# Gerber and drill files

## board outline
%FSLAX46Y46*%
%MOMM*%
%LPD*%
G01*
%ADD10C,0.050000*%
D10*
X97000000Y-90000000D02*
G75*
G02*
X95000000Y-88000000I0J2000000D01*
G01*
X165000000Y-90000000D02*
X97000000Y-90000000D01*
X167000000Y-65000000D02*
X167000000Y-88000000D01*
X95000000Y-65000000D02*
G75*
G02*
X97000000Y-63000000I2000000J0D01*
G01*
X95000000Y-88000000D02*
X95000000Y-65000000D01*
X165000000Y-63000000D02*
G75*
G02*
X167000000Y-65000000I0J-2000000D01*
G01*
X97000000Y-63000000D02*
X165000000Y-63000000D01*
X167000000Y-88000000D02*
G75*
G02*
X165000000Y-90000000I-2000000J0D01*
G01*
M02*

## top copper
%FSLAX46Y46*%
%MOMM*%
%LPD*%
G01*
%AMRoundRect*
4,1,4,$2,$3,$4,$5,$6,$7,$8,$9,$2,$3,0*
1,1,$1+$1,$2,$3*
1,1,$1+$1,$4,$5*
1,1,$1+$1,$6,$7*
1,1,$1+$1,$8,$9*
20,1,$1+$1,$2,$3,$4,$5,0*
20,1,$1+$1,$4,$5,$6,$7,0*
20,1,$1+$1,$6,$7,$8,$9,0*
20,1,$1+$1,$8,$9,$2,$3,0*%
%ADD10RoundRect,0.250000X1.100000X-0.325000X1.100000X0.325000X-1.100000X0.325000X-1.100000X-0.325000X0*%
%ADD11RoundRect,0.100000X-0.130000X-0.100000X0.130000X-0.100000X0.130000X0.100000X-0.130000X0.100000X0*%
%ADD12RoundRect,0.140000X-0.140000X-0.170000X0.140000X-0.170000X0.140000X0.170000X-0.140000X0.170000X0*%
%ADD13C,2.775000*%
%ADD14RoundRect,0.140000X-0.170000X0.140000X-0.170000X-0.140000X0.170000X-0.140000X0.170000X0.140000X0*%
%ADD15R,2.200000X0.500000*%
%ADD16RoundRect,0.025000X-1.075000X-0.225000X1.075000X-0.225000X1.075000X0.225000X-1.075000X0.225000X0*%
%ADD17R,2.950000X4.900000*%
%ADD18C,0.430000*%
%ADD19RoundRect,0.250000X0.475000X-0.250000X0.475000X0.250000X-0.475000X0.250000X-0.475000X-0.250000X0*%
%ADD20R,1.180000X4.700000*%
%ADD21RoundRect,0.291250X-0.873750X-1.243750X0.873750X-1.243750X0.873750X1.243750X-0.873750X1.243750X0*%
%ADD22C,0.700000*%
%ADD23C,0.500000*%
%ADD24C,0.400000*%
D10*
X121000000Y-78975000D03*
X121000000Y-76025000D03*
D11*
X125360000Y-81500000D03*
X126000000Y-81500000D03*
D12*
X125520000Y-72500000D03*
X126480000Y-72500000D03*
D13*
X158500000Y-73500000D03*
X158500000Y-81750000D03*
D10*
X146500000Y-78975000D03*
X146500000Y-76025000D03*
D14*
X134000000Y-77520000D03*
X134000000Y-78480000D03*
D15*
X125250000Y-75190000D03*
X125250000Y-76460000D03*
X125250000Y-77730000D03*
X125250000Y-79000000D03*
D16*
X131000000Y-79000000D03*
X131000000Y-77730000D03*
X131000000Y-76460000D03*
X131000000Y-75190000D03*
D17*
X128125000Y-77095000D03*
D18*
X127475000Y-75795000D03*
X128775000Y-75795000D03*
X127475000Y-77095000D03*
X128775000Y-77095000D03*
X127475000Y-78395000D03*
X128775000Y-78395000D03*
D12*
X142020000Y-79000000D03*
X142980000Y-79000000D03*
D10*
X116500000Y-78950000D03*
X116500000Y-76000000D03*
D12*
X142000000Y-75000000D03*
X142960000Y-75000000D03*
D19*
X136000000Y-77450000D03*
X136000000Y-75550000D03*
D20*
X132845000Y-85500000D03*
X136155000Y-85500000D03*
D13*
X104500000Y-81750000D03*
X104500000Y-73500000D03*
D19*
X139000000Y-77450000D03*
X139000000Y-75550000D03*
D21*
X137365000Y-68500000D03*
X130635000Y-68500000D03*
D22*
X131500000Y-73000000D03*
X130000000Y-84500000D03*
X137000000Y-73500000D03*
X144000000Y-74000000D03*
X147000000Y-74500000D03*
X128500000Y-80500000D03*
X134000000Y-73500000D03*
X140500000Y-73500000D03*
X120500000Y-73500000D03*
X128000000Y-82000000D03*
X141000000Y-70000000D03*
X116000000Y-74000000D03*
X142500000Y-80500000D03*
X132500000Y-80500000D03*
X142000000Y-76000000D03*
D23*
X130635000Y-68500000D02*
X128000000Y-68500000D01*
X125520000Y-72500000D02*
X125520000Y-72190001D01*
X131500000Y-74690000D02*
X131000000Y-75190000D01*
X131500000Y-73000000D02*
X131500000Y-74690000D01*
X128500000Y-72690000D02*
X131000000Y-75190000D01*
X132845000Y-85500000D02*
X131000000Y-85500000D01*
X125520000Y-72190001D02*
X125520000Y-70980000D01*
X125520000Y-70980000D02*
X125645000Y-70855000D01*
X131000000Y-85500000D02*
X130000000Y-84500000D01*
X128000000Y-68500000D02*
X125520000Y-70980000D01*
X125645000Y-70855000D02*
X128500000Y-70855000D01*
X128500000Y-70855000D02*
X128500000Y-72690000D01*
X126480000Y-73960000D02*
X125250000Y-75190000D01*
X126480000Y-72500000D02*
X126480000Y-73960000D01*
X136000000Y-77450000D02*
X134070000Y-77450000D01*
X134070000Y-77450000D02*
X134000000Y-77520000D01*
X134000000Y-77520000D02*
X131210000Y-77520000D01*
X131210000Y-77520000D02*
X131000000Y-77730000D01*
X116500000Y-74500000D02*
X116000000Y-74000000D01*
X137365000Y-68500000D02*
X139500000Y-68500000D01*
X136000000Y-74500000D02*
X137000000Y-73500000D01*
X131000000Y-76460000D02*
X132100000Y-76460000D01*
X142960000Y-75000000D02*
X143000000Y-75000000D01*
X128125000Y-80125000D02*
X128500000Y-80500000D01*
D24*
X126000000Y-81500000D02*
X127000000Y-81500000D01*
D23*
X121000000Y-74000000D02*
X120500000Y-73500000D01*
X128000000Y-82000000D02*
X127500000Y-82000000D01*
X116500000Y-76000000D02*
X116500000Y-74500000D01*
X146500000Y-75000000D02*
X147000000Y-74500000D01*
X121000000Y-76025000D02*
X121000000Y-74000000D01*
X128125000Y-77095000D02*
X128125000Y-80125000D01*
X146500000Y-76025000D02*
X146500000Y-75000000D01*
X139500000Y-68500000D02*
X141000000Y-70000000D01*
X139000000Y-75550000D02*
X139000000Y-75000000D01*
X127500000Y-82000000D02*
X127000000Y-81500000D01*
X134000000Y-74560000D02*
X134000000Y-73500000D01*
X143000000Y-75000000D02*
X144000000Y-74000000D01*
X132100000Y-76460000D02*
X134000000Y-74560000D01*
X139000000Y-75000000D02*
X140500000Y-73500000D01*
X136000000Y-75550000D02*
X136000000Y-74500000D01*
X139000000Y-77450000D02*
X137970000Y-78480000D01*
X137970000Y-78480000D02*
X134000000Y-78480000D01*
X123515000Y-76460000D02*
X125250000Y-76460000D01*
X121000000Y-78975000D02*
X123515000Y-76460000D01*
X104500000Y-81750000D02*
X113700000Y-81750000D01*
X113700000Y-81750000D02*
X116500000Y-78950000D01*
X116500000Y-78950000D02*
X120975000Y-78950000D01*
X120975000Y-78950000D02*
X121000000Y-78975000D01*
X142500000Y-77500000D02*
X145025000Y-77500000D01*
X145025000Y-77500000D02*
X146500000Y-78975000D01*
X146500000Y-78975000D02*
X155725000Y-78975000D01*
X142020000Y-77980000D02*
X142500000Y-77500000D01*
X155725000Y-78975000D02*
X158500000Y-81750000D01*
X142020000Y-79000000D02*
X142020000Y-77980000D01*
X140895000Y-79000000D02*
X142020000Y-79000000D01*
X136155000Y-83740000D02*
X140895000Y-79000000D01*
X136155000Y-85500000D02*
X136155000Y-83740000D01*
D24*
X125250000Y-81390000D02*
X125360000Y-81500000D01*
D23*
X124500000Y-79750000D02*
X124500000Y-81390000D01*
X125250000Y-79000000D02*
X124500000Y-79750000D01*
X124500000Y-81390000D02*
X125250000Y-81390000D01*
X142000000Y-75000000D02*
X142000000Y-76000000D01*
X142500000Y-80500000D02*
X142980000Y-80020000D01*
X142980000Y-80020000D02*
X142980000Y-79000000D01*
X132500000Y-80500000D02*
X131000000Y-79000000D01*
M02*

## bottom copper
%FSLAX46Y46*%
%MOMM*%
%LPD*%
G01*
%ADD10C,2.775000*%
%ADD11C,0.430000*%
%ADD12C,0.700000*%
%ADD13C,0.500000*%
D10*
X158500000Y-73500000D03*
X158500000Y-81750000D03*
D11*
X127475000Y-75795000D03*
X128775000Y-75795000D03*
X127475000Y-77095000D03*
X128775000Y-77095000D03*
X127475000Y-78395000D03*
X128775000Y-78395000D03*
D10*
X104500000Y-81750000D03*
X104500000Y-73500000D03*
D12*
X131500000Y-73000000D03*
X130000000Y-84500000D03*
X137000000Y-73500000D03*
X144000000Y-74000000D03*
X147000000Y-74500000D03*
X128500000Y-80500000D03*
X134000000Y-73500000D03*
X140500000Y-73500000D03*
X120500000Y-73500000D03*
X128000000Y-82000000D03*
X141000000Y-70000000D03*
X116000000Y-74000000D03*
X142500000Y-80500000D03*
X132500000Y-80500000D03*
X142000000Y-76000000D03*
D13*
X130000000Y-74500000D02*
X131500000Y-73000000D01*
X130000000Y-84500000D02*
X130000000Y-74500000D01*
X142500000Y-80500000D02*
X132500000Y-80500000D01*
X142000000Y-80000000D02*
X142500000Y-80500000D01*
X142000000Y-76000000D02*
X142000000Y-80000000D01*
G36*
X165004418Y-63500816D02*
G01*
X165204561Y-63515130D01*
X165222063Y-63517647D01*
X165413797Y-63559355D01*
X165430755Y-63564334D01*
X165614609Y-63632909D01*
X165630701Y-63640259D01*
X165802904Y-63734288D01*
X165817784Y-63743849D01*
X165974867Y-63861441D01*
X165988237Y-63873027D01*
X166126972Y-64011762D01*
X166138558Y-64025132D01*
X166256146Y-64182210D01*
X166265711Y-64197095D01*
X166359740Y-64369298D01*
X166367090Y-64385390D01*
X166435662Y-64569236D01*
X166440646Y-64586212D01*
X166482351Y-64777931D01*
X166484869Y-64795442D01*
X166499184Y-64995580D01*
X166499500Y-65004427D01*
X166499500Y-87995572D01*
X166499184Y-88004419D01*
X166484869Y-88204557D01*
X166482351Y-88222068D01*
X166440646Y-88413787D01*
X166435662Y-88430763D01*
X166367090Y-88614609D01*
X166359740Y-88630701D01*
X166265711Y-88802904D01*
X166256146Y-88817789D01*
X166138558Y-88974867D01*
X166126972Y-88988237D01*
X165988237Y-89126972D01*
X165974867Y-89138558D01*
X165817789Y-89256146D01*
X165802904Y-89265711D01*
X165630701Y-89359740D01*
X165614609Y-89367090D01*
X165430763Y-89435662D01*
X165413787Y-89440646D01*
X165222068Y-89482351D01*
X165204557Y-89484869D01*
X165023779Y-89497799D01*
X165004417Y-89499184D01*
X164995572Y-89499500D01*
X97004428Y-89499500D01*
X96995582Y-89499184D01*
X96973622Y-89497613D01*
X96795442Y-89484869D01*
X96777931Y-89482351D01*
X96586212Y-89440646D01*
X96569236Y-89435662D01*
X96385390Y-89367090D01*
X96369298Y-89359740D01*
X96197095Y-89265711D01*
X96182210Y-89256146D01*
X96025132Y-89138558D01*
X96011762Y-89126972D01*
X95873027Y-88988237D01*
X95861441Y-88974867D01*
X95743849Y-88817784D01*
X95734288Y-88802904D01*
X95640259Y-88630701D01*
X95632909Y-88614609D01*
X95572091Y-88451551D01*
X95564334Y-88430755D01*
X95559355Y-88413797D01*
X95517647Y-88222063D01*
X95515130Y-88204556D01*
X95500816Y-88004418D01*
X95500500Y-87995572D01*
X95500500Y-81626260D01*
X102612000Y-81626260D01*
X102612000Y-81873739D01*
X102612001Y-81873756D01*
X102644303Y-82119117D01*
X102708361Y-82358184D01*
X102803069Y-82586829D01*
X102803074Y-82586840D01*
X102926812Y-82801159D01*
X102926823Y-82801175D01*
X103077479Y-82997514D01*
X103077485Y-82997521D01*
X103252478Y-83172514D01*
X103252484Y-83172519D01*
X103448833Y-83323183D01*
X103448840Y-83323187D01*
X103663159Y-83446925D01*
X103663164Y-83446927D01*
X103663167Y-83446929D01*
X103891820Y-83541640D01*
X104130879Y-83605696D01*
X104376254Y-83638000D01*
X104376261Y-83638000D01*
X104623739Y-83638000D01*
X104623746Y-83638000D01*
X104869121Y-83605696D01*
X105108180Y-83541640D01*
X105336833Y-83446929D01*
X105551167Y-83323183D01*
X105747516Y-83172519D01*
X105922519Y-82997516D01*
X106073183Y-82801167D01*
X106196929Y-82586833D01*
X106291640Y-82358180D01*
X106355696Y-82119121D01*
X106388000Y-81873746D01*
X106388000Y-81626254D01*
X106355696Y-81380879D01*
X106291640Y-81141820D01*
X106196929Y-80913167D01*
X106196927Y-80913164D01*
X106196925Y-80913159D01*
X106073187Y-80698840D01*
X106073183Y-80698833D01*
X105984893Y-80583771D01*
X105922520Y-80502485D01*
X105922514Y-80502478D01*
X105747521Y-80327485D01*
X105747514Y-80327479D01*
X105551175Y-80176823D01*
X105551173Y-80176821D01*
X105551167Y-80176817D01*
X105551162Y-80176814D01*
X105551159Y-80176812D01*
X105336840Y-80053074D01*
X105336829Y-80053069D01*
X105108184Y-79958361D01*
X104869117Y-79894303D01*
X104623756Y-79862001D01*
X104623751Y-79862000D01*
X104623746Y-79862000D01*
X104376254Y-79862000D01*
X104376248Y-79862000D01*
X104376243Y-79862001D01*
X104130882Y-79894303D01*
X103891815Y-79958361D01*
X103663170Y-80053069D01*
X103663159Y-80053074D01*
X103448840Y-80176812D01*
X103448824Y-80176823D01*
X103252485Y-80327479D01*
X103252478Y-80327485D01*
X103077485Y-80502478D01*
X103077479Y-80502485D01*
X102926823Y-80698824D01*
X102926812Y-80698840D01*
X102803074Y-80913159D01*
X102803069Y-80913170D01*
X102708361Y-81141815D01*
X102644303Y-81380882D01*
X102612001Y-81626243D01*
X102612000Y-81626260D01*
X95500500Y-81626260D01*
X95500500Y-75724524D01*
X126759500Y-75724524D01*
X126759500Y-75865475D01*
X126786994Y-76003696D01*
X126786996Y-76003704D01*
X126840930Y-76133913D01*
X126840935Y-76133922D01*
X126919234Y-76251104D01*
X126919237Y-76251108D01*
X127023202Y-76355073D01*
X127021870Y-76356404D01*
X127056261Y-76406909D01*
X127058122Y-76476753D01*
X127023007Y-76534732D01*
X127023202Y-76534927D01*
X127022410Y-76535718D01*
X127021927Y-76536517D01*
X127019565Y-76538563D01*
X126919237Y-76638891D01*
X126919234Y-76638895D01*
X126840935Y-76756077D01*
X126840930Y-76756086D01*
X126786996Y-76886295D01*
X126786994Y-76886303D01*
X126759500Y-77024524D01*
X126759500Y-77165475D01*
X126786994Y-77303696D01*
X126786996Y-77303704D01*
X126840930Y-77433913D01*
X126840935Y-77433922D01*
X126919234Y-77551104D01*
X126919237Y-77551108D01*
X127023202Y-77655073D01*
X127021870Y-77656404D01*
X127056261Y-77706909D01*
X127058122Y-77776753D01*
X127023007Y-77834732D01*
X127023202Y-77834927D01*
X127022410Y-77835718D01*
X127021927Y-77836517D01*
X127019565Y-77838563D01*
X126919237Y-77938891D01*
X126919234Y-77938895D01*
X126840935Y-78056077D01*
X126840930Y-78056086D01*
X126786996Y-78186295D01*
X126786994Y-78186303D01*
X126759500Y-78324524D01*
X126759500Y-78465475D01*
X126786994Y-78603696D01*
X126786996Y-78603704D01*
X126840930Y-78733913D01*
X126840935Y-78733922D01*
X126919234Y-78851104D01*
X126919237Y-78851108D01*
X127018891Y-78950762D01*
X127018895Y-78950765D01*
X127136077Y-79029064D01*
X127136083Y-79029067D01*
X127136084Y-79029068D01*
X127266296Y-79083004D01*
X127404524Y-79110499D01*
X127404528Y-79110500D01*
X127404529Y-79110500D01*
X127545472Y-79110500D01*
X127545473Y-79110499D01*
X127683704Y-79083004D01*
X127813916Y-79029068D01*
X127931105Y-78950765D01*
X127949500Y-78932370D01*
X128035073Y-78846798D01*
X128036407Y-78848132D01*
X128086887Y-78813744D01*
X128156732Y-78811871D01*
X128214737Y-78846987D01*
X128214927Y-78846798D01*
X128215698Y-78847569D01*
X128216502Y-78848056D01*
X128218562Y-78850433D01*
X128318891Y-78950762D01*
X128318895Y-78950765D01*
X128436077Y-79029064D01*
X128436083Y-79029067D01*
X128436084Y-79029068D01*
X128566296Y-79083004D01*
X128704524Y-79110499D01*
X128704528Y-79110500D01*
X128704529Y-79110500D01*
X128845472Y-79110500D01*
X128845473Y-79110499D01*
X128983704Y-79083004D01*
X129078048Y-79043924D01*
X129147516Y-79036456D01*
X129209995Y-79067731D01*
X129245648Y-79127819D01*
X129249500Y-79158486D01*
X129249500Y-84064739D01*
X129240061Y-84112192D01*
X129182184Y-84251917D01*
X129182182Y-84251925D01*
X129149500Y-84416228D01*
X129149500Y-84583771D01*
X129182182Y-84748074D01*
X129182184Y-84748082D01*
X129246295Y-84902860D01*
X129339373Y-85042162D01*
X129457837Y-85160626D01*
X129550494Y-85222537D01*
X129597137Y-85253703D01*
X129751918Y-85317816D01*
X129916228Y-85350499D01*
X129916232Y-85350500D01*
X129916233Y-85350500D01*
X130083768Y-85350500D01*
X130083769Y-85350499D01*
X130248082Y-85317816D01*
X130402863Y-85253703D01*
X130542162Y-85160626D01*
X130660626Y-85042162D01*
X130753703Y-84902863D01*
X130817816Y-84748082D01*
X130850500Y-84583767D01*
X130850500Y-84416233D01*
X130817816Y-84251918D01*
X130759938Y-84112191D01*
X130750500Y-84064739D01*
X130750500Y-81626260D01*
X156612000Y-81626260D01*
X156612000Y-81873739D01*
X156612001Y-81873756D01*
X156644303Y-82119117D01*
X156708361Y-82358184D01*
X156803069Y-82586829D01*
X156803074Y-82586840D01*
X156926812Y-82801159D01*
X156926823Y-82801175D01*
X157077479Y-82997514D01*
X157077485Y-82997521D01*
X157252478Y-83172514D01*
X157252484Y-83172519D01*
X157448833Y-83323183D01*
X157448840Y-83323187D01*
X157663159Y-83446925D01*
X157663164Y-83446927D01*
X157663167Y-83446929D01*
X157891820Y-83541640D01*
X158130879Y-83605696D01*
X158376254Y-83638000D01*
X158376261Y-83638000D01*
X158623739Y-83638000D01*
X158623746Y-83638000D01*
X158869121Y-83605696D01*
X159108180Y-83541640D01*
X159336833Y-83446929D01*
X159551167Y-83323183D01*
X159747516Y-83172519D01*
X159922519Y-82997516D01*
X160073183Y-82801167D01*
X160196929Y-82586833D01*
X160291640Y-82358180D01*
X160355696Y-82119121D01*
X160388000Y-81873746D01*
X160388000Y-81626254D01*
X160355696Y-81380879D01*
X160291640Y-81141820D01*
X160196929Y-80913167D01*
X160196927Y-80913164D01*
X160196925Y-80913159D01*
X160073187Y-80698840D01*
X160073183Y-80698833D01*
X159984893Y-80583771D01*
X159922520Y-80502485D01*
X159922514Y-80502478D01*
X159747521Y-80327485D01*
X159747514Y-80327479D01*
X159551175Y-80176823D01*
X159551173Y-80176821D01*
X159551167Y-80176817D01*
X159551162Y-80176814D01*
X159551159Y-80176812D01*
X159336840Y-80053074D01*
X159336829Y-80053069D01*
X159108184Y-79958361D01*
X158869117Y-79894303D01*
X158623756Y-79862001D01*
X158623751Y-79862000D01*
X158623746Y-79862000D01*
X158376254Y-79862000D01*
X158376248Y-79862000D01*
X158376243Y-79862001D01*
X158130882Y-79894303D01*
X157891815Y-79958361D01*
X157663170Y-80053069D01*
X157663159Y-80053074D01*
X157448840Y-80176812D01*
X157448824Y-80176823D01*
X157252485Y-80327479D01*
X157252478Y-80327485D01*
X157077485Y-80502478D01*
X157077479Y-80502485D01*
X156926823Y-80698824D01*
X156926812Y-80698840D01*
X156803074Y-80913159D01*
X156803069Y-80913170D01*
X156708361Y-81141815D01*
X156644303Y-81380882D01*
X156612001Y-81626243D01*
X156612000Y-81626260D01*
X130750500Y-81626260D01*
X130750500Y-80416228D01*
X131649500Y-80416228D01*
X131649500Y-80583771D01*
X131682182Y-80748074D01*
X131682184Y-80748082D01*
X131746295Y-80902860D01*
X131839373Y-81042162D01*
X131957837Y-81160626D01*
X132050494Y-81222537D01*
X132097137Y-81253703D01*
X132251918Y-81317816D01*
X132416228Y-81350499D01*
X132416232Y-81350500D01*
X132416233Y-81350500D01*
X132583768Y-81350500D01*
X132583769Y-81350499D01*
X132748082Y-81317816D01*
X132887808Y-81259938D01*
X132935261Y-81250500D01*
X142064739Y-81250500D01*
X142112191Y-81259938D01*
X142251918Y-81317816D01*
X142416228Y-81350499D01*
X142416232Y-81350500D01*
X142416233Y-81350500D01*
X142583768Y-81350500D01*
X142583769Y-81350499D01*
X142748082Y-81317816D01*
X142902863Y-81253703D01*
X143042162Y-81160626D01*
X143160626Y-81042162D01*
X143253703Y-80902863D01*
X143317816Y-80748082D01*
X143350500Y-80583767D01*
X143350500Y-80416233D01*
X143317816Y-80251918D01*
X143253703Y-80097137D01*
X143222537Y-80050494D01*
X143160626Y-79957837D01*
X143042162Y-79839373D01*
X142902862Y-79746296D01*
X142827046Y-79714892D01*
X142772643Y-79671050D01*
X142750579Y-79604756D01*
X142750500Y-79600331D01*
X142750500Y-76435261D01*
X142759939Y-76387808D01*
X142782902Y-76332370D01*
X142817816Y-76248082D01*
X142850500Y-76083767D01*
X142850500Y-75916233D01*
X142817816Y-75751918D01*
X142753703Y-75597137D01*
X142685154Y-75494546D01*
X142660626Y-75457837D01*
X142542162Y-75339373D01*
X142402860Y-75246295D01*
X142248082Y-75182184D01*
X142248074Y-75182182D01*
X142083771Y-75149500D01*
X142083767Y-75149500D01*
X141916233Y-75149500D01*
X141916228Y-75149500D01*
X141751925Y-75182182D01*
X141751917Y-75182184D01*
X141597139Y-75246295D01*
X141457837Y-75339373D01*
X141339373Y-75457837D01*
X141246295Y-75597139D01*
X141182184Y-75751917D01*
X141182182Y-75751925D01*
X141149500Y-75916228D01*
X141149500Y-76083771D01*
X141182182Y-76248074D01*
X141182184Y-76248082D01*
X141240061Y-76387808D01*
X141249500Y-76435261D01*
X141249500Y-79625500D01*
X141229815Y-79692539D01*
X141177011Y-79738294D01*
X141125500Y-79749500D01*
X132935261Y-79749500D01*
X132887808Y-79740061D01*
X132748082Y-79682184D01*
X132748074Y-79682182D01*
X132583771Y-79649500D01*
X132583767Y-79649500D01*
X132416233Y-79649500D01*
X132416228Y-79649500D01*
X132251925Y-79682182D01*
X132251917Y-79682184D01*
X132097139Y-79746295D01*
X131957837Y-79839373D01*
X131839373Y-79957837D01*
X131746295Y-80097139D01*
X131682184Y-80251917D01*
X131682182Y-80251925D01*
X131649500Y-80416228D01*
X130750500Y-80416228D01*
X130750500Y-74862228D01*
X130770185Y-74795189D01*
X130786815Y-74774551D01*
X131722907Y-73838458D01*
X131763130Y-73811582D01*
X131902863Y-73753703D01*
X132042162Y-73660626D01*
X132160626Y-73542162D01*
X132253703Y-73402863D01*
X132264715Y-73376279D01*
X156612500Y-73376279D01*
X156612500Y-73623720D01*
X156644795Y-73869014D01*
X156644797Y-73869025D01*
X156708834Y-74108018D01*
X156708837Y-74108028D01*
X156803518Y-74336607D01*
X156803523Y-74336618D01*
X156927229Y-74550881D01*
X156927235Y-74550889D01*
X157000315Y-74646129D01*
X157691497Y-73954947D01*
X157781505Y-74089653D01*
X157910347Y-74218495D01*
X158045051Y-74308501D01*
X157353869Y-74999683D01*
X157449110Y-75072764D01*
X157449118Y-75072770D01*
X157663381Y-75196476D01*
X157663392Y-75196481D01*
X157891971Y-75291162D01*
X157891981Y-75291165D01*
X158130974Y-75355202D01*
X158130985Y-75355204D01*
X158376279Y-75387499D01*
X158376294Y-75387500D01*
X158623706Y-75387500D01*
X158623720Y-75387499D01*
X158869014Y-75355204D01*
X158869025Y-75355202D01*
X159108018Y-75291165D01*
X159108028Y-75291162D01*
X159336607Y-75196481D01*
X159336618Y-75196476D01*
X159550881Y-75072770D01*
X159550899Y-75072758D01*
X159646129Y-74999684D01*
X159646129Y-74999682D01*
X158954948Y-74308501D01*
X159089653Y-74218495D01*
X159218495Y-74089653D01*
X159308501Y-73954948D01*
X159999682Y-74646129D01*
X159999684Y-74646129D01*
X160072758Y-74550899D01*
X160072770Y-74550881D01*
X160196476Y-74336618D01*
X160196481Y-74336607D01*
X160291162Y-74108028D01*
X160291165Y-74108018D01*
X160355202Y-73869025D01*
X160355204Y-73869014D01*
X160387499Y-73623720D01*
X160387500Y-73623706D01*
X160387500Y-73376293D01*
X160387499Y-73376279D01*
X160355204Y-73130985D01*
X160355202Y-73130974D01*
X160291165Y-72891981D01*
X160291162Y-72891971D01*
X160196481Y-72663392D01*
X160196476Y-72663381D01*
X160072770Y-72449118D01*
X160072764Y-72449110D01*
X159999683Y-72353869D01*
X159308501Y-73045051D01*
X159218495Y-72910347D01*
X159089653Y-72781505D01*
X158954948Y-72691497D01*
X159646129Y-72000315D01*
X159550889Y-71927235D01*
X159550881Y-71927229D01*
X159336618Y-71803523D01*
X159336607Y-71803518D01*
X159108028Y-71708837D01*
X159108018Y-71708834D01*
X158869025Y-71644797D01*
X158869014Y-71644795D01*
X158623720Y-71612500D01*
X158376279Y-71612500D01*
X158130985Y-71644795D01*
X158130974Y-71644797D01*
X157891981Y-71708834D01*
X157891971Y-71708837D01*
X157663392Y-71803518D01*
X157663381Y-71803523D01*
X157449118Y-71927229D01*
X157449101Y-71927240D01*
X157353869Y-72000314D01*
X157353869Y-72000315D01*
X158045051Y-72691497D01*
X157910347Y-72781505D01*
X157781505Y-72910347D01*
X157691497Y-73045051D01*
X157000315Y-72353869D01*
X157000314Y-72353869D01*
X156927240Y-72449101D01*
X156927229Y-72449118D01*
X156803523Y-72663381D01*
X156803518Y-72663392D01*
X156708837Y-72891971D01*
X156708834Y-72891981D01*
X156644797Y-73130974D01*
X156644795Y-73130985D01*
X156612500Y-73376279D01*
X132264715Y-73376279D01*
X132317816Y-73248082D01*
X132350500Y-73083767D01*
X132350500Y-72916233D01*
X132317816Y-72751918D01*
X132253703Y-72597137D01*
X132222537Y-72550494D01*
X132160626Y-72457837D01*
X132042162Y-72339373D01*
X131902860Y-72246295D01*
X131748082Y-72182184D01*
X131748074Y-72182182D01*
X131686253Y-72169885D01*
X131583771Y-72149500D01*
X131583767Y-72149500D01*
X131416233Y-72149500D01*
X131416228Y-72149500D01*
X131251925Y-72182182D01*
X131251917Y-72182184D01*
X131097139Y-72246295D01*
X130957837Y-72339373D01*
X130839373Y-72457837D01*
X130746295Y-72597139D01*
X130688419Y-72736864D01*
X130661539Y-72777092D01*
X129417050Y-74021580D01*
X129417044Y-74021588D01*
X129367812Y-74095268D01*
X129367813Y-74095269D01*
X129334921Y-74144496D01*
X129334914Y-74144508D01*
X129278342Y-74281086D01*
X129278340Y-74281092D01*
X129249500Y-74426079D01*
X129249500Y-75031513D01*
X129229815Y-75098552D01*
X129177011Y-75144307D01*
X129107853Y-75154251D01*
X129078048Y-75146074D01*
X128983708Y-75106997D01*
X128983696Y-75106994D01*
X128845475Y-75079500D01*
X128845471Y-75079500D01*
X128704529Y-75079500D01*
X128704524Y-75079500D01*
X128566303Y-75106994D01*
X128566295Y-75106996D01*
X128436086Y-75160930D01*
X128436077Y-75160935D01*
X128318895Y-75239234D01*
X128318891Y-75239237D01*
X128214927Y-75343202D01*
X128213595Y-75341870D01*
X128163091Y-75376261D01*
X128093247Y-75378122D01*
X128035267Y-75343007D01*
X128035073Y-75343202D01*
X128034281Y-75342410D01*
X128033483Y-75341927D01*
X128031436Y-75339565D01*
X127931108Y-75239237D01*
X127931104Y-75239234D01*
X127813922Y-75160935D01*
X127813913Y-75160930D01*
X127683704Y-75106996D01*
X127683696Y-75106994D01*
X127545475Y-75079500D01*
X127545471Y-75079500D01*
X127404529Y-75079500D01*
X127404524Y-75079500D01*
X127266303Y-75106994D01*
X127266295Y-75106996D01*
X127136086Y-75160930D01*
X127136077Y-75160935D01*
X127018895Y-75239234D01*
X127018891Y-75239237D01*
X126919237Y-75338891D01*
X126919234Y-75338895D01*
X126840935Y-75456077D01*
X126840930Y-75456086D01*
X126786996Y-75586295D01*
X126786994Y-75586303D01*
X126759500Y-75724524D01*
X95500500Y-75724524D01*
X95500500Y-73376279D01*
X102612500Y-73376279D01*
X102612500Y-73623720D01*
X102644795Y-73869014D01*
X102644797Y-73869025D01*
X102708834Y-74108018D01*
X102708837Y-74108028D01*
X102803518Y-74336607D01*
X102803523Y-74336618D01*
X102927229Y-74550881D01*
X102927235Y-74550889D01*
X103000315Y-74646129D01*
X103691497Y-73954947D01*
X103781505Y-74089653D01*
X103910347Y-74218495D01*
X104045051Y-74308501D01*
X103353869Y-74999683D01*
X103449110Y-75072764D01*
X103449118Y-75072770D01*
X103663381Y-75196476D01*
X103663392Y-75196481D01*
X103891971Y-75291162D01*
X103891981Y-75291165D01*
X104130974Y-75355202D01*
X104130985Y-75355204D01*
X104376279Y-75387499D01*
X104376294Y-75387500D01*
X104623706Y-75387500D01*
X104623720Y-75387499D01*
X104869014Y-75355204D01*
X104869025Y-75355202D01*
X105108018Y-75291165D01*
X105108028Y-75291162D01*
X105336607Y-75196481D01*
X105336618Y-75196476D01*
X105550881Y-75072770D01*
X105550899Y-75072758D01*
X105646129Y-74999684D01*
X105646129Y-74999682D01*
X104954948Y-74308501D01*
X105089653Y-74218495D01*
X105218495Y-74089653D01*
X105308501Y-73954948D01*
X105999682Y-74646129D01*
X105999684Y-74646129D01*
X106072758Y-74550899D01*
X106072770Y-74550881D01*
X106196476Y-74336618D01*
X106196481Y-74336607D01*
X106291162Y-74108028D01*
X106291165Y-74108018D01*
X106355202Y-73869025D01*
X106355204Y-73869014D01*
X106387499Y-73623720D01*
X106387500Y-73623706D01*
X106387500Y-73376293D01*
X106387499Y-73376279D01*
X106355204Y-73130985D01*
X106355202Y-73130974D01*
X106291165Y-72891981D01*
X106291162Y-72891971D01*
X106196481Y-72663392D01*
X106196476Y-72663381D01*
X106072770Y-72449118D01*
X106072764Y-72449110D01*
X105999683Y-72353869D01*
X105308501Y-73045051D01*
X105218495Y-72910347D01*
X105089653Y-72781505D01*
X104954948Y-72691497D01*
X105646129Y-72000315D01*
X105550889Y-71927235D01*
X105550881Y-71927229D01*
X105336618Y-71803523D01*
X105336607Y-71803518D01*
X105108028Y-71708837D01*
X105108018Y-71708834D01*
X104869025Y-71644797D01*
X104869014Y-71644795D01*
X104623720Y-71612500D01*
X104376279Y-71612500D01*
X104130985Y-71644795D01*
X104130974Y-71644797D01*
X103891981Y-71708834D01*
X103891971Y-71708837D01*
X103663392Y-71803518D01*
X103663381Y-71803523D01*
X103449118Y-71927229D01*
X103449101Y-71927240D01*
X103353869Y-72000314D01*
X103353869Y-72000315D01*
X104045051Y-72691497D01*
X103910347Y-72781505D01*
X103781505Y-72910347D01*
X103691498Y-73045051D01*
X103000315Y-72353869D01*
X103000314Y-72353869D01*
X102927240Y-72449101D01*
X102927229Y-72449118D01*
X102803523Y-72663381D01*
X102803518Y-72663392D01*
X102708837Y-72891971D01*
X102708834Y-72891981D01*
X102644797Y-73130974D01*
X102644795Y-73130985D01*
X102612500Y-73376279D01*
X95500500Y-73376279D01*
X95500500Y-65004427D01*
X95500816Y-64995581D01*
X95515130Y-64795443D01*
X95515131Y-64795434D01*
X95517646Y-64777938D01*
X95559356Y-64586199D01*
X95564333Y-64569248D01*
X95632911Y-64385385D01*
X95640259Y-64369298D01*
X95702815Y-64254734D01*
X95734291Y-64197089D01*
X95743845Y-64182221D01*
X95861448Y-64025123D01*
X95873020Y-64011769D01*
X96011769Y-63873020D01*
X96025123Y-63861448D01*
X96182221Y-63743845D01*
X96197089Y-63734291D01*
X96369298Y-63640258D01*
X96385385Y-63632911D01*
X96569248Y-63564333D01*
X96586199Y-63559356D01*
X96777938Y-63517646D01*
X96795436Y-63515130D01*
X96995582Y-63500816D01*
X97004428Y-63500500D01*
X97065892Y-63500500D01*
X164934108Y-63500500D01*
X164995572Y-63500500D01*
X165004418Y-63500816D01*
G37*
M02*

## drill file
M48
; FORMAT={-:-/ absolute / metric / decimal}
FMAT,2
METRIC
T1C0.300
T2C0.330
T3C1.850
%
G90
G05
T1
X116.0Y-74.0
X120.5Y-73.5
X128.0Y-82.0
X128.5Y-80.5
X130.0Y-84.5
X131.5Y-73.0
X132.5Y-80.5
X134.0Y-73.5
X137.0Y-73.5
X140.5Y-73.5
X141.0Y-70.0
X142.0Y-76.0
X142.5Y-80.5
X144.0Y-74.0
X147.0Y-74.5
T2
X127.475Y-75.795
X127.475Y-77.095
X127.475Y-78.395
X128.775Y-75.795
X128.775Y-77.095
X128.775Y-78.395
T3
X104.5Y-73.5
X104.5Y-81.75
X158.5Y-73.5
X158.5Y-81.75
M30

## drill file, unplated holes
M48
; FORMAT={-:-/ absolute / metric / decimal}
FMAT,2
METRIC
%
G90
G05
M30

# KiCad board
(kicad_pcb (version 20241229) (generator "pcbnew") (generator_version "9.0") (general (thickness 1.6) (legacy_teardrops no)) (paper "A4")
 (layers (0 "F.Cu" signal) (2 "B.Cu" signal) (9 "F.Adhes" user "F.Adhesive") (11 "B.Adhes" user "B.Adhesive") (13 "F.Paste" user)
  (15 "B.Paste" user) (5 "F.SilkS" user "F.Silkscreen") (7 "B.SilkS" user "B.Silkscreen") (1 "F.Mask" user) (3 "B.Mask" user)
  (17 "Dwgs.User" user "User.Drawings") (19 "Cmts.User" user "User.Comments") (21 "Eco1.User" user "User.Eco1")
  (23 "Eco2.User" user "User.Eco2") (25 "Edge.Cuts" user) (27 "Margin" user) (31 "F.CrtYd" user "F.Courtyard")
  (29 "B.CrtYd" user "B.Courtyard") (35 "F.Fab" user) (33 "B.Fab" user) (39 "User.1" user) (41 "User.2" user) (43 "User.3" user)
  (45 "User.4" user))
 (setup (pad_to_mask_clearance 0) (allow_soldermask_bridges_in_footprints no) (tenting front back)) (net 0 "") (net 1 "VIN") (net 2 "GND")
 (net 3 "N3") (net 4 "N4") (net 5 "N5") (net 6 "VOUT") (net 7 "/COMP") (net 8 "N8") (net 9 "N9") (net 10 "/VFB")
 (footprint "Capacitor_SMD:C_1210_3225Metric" (layer "F.Cu") (at 121 77.5 90)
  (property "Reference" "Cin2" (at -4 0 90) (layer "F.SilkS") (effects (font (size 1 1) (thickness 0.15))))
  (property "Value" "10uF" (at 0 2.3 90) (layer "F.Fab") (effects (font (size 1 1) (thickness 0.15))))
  (pad "1" smd roundrect (at -1.475 0 90) (size 1.15 2.7) (layers "F.Cu" "F.Mask" "F.Paste") (roundrect_rratio 0.217391) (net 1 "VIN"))
  (pad "2" smd roundrect (at 1.475 0 90) (size 1.15 2.7) (layers "F.Cu" "F.Mask" "F.Paste") (roundrect_rratio 0.217391) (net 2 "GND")))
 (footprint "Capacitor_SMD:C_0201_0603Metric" (layer "F.Cu") (at 125.68 81.5)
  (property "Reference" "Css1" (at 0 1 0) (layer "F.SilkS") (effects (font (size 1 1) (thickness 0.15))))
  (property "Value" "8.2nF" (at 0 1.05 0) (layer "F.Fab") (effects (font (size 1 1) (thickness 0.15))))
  (pad "" smd roundrect (at -0.345 0) (size 0.318 0.36) (layers "F.Paste") (roundrect_rratio 0.25))
  (pad "" smd roundrect (at 0.345 0) (size 0.318 0.36) (layers "F.Paste") (roundrect_rratio 0.25))
  (pad "1" smd roundrect (at -0.32 0) (size 0.46 0.4) (layers "F.Cu" "F.Mask") (roundrect_rratio 0.25) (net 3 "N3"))
  (pad "2" smd roundrect (at 0.32 0) (size 0.46 0.4) (layers "F.Cu" "F.Mask") (roundrect_rratio 0.25) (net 2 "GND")))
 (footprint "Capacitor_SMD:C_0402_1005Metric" (layer "F.Cu") (at 126 72.5)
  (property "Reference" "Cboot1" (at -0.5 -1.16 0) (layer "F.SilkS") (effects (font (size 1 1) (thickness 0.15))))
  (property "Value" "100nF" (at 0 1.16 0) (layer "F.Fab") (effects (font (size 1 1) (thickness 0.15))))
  (pad "1" smd roundrect (at -0.48 0) (size 0.56 0.62) (layers "F.Cu" "F.Mask" "F.Paste") (roundrect_rratio 0.25) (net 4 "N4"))
  (pad "2" smd roundrect (at 0.48 0) (size 0.56 0.62) (layers "F.Cu" "F.Mask" "F.Paste") (roundrect_rratio 0.25) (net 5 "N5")))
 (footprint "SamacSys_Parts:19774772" (layer "F.Cu") (at 158.5 73.5 -90)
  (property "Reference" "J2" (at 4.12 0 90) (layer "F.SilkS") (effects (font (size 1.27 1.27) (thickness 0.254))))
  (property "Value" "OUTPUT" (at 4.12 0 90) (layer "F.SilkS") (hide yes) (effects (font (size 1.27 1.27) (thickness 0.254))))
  (pad "1" thru_hole circle (at 0 0 270) (size 2.775 2.775) (drill 1.85) (layers "*.Cu" "*.Mask") (remove_unused_layers no) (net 2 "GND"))
  (pad "2" thru_hole circle (at 8.25 0 270) (size 2.775 2.775) (drill 1.85) (layers "*.Cu" "*.Mask") (remove_unused_layers no)
   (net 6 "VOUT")))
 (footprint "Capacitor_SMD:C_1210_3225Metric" (layer "F.Cu") (at 146.5 77.5 90)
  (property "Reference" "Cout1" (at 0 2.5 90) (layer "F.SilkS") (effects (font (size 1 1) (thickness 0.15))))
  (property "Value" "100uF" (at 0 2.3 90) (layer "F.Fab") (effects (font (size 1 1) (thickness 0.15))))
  (pad "1" smd roundrect (at -1.475 0 90) (size 1.15 2.7) (layers "F.Cu" "F.Mask" "F.Paste") (roundrect_rratio 0.217391) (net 6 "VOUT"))
  (pad "2" smd roundrect (at 1.475 0 90) (size 1.15 2.7) (layers "F.Cu" "F.Mask" "F.Paste") (roundrect_rratio 0.217391) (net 2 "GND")))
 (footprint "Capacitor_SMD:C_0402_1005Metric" (layer "F.Cu") (at 134 78 -90)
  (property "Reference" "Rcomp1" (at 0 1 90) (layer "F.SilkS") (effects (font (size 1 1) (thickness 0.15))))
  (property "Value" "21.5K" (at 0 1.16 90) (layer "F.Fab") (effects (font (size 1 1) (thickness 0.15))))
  (pad "1" smd roundrect (at -0.48 0 270) (size 0.56 0.62) (layers "F.Cu" "F.Mask" "F.Paste") (roundrect_rratio 0.25) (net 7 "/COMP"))
  (pad "2" smd roundrect (at 0.48 0 270) (size 0.56 0.62) (layers "F.Cu" "F.Mask" "F.Paste") (roundrect_rratio 0.25) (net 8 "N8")))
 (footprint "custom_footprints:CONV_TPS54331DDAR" (layer "F.Cu") (at 128.125 77.095)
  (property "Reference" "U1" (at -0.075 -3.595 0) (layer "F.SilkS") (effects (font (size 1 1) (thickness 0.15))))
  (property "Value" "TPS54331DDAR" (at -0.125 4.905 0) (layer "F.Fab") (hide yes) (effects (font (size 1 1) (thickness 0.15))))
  (pad "1" smd rect (at -2.875 -1.905) (size 2.2 0.5) (layers "F.Cu") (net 5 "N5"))
  (pad "2" smd rect (at -2.875 -0.635) (size 2.2 0.5) (layers "F.Cu") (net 1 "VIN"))
  (pad "3" smd rect (at -2.875 0.635) (size 2.2 0.5) (layers "F.Cu") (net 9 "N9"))
  (pad "4" smd rect (at -2.875 1.905) (size 2.2 0.5) (layers "F.Cu") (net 3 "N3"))
  (pad "5" smd roundrect (at 2.875 1.905) (size 2.2 0.5) (layers "F.Cu") (roundrect_rratio 0.05) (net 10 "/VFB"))
  (pad "6" smd roundrect (at 2.875 0.635) (size 2.2 0.5) (layers "F.Cu") (roundrect_rratio 0.05) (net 7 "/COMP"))
  (pad "7" smd roundrect (at 2.875 -0.635) (size 2.2 0.5) (layers "F.Cu") (roundrect_rratio 0.05) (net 2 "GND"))
  (pad "8" smd roundrect (at 2.875 -1.905) (size 2.2 0.5) (layers "F.Cu") (roundrect_rratio 0.05) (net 4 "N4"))
  (pad "9" smd rect (at 0 0) (size 2.95 4.9) (layers "F.Cu") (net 2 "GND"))
  (pad "10" thru_hole circle (at -0.65 -1.3) (size 0.43 0.43) (drill 0.33) (layers "*.Cu") (remove_unused_layers no))
  (pad "11" thru_hole circle (at 0.65 -1.3) (size 0.43 0.43) (drill 0.33) (layers "*.Cu") (remove_unused_layers no))
  (pad "12" thru_hole circle (at -0.65 0) (size 0.43 0.43) (drill 0.33) (layers "*.Cu") (remove_unused_layers no))
  (pad "13" thru_hole circle (at 0.65 0) (size 0.43 0.43) (drill 0.33) (layers "*.Cu") (remove_unused_layers no))
  (pad "14" thru_hole circle (at -0.65 1.3) (size 0.43 0.43) (drill 0.33) (layers "*.Cu") (remove_unused_layers no))
  (pad "15" thru_hole circle (at 0.65 1.3) (size 0.43 0.43) (drill 0.33) (layers "*.Cu") (remove_unused_layers no)))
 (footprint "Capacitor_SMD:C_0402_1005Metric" (layer "F.Cu") (at 142.5 79)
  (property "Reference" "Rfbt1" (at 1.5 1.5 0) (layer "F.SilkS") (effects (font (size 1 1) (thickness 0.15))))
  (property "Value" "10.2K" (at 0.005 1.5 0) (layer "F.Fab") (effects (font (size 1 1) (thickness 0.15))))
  (pad "1" smd roundrect (at -0.48 0) (size 0.56 0.62) (layers "F.Cu" "F.Mask" "F.Paste") (roundrect_rratio 0.25) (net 6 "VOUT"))
  (pad "2" smd roundrect (at 0.48 0) (size 0.56 0.62) (layers "F.Cu" "F.Mask" "F.Paste") (roundrect_rratio 0.25) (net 10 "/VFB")))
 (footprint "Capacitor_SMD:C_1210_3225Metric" (layer "F.Cu") (at 116.5 77.475 90)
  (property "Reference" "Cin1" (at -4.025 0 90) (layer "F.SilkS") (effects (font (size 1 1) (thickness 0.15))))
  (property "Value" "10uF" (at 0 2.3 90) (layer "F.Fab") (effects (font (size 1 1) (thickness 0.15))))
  (pad "1" smd roundrect (at -1.475 0 90) (size 1.15 2.7) (layers "F.Cu" "F.Mask" "F.Paste") (roundrect_rratio 0.217391) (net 1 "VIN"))
  (pad "2" smd roundrect (at 1.475 0 90) (size 1.15 2.7) (layers "F.Cu" "F.Mask" "F.Paste") (roundrect_rratio 0.217391) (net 2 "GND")))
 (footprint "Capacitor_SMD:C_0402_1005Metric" (layer "F.Cu") (at 142.48 75)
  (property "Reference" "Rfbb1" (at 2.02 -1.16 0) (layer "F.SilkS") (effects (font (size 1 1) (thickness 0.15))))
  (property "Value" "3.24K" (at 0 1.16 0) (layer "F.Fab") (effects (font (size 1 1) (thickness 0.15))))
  (pad "1" smd roundrect (at -0.48 0) (size 0.56 0.62) (layers "F.Cu" "F.Mask" "F.Paste") (roundrect_rratio 0.25) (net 10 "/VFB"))
  (pad "2" smd roundrect (at 0.48 0) (size 0.56 0.62) (layers "F.Cu" "F.Mask" "F.Paste") (roundrect_rratio 0.25) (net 2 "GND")))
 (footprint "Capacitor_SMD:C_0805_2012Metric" (layer "F.Cu") (at 136 76.5 90)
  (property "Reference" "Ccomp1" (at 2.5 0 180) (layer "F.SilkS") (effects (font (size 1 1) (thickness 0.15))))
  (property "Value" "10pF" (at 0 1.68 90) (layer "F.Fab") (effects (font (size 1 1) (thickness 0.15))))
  (pad "1" smd roundrect (at -0.95 0 90) (size 1 1.45) (layers "F.Cu" "F.Mask" "F.Paste") (roundrect_rratio 0.25) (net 7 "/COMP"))
  (pad "2" smd roundrect (at 0.95 0 90) (size 1 1.45) (layers "F.Cu" "F.Mask" "F.Paste") (roundrect_rratio 0.25) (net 2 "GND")))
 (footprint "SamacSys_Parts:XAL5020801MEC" (layer "F.Cu") (at 134.5 85.5)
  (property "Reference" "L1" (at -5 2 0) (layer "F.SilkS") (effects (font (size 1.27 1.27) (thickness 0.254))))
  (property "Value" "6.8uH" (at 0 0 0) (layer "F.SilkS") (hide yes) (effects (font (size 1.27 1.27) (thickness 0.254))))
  (pad "1" smd rect (at -1.655 0) (size 1.18 4.7) (layers "F.Cu" "F.Mask" "F.Paste") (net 4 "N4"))
  (pad "2" smd rect (at 1.655 0) (size 1.18 4.7) (layers "F.Cu" "F.Mask" "F.Paste") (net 6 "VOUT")))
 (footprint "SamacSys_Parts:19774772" (layer "F.Cu") (at 104.5 81.75 90)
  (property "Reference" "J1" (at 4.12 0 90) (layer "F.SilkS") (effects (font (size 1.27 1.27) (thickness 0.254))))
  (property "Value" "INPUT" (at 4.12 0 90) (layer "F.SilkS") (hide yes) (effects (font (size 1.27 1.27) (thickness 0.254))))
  (pad "1" thru_hole circle (at 0 0 90) (size 2.775 2.775) (drill 1.85) (layers "*.Cu" "*.Mask") (remove_unused_layers no) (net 1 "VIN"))
  (pad "2" thru_hole circle (at 8.25 0 90) (size 2.775 2.775) (drill 1.85) (layers "*.Cu" "*.Mask") (remove_unused_layers no) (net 2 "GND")))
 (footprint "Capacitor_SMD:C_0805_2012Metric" (layer "F.Cu") (at 139 76.5 90)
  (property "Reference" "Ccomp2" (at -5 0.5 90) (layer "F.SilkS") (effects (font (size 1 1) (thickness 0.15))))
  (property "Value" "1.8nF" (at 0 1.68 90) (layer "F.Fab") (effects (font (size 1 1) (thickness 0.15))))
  (pad "1" smd roundrect (at -0.95 0 90) (size 1 1.45) (layers "F.Cu" "F.Mask" "F.Paste") (roundrect_rratio 0.25) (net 8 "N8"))
  (pad "2" smd roundrect (at 0.95 0 90) (size 1 1.45) (layers "F.Cu" "F.Mask" "F.Paste") (roundrect_rratio 0.25) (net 2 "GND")))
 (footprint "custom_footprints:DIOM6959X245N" (layer "F.Cu") (at 134 68.5)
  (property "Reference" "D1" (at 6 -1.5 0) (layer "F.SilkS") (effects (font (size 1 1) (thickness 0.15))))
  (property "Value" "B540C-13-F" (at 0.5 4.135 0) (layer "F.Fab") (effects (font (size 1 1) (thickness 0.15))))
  (pad "A" smd roundrect (at 3.365 0) (size 2.33 3.07) (layers "F.Cu" "F.Mask" "F.Paste") (roundrect_rratio 0.125) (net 2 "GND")
   (solder_mask_margin 0.102))
  (pad "C" smd roundrect (at -3.365 0) (size 2.33 3.07) (layers "F.Cu" "F.Mask" "F.Paste") (roundrect_rratio 0.125) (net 4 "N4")
   (solder_mask_margin 0.102)))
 (gr_arc (start 97 90) (mid 95.585786 89.414214) (end 95 88) (stroke (width 0.05) (type default)) (layer "Edge.Cuts"))
 (gr_line (start 165 90) (end 97 90) (stroke (width 0.05) (type default)) (layer "Edge.Cuts"))
 (gr_line (start 167 65) (end 167 88) (stroke (width 0.05) (type default)) (layer "Edge.Cuts"))
 (gr_arc (start 95 65) (mid 95.585786 63.585786) (end 97 63) (stroke (width 0.05) (type default)) (layer "Edge.Cuts"))
 (gr_line (start 95 88) (end 95 65) (stroke (width 0.05) (type default)) (layer "Edge.Cuts"))
 (gr_arc (start 165 63) (mid 166.414214 63.585786) (end 167 65) (stroke (width 0.05) (type default)) (layer "Edge.Cuts"))
 (gr_line (start 97 63) (end 165 63) (stroke (width 0.05) (type default)) (layer "Edge.Cuts"))
 (gr_arc (start 167 88) (mid 166.414214 89.414214) (end 165 90) (stroke (width 0.05) (type default)) (layer "Edge.Cuts"))
 (segment (start 130.635 68.5) (end 128 68.5) (width 0.5) (layer "F.Cu") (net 4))
 (segment (start 125.52 72.5) (end 125.52 72.190001) (width 0.5) (layer "F.Cu") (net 4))
 (segment (start 131.5 74.69) (end 131 75.19) (width 0.5) (layer "F.Cu") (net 4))
 (segment (start 131.5 73) (end 131.5 74.69) (width 0.5) (layer "F.Cu") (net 4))
 (segment (start 128.5 72.69) (end 131 75.19) (width 0.5) (layer "F.Cu") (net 4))
 (segment (start 132.845 85.5) (end 131 85.5) (width 0.5) (layer "F.Cu") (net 4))
 (segment (start 125.52 72.190001) (end 125.52 70.98) (width 0.5) (layer "F.Cu") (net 4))
 (segment (start 125.52 70.98) (end 125.645 70.855) (width 0.5) (layer "F.Cu") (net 4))
 (segment (start 131 85.5) (end 130 84.5) (width 0.5) (layer "F.Cu") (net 4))
 (segment (start 128 68.5) (end 125.52 70.98) (width 0.5) (layer "F.Cu") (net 4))
 (segment (start 125.645 70.855) (end 128.5 70.855) (width 0.5) (layer "F.Cu") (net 4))
 (segment (start 128.5 70.855) (end 128.5 72.69) (width 0.5) (layer "F.Cu") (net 4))
 (via (at 131.5 73) (size 0.7) (drill 0.3) (layers "F.Cu" "B.Cu") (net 4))
 (via (at 130 84.5) (size 0.7) (drill 0.3) (layers "F.Cu" "B.Cu") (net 4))
 (segment (start 130 74.5) (end 131.5 73) (width 0.5) (layer "B.Cu") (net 4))
 (segment (start 130 84.5) (end 130 74.5) (width 0.5) (layer "B.Cu") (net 4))
 (segment (start 126.48 73.96) (end 125.25 75.19) (width 0.5) (layer "F.Cu") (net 5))
 (segment (start 126.48 72.5) (end 126.48 73.96) (width 0.5) (layer "F.Cu") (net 5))
 (segment (start 136 77.45) (end 134.07 77.45) (width 0.5) (layer "F.Cu") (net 7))
 (segment (start 134.07 77.45) (end 134 77.52) (width 0.5) (layer "F.Cu") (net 7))
 (segment (start 134 77.52) (end 131.21 77.52) (width 0.5) (layer "F.Cu") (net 7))
 (segment (start 131.21 77.52) (end 131 77.73) (width 0.5) (layer "F.Cu") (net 7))
 (segment (start 116.5 74.5) (end 116 74) (width 0.5) (layer "F.Cu") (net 2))
 (segment (start 137.365 68.5) (end 139.5 68.5) (width 0.5) (layer "F.Cu") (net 2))
 (segment (start 136 74.5) (end 137 73.5) (width 0.5) (layer "F.Cu") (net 2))
 (segment (start 131 76.46) (end 132.1 76.46) (width 0.5) (layer "F.Cu") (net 2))
 (segment (start 142.96 75) (end 143 75) (width 0.5) (layer "F.Cu") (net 2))
 (segment (start 128.125 80.125) (end 128.5 80.5) (width 0.5) (layer "F.Cu") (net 2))
 (segment (start 126 81.5) (end 127 81.5) (width 0.4) (layer "F.Cu") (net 2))
 (segment (start 121 74) (end 120.5 73.5) (width 0.5) (layer "F.Cu") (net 2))
 (segment (start 128 82) (end 127.5 82) (width 0.5) (layer "F.Cu") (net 2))
 (segment (start 116.5 76) (end 116.5 74.5) (width 0.5) (layer "F.Cu") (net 2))
 (segment (start 146.5 75) (end 147 74.5) (width 0.5) (layer "F.Cu") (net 2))
 (segment (start 121 76.025) (end 121 74) (width 0.5) (layer "F.Cu") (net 2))
 (segment (start 128.125 77.095) (end 128.125 80.125) (width 0.5) (layer "F.Cu") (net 2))
 (segment (start 146.5 76.025) (end 146.5 75) (width 0.5) (layer "F.Cu") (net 2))
 (segment (start 139.5 68.5) (end 141 70) (width 0.5) (layer "F.Cu") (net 2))
 (segment (start 139 75.55) (end 139 75) (width 0.5) (layer "F.Cu") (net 2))
 (segment (start 127.5 82) (end 127 81.5) (width 0.5) (layer "F.Cu") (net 2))
 (segment (start 134 74.56) (end 134 73.5) (width 0.5) (layer "F.Cu") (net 2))
 (segment (start 143 75) (end 144 74) (width 0.5) (layer "F.Cu") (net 2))
 (segment (start 132.1 76.46) (end 134 74.56) (width 0.5) (layer "F.Cu") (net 2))
 (segment (start 139 75) (end 140.5 73.5) (width 0.5) (layer "F.Cu") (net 2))
 (segment (start 136 75.55) (end 136 74.5) (width 0.5) (layer "F.Cu") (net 2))
 (via (at 137 73.5) (size 0.7) (drill 0.3) (layers "F.Cu" "B.Cu") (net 2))
 (via (at 144 74) (size 0.7) (drill 0.3) (layers "F.Cu" "B.Cu") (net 2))
 (via (at 147 74.5) (size 0.7) (drill 0.3) (layers "F.Cu" "B.Cu") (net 2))
 (via (at 128.5 80.5) (size 0.7) (drill 0.3) (layers "F.Cu" "B.Cu") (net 2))
 (via (at 134 73.5) (size 0.7) (drill 0.3) (layers "F.Cu" "B.Cu") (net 2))
 (via (at 140.5 73.5) (size 0.7) (drill 0.3) (layers "F.Cu" "B.Cu") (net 2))
 (via (at 120.5 73.5) (size 0.7) (drill 0.3) (layers "F.Cu" "B.Cu") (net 2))
 (via (at 128 82) (size 0.7) (drill 0.3) (layers "F.Cu" "B.Cu") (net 2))
 (via (at 141 70) (size 0.7) (drill 0.3) (layers "F.Cu" "B.Cu") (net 2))
 (via (at 116 74) (size 0.7) (drill 0.3) (layers "F.Cu" "B.Cu") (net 2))
 (segment (start 139 77.45) (end 137.97 78.48) (width 0.5) (layer "F.Cu") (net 8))
 (segment (start 137.97 78.48) (end 134 78.48) (width 0.5) (layer "F.Cu") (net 8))
 (segment (start 123.515 76.46) (end 125.25 76.46) (width 0.5) (layer "F.Cu") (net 1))
 (segment (start 121 78.975) (end 123.515 76.46) (width 0.5) (layer "F.Cu") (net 1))
 (segment (start 104.5 81.75) (end 113.7 81.75) (width 0.5) (layer "F.Cu") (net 1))
 (segment (start 113.7 81.75) (end 116.5 78.95) (width 0.5) (layer "F.Cu") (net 1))
 (segment (start 116.5 78.95) (end 120.975 78.95) (width 0.5) (layer "F.Cu") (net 1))
 (segment (start 120.975 78.95) (end 121 78.975) (width 0.5) (layer "F.Cu") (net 1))
 (segment (start 142.5 77.5) (end 145.025 77.5) (width 0.5) (layer "F.Cu") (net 6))
 (segment (start 145.025 77.5) (end 146.5 78.975) (width 0.5) (layer "F.Cu") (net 6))
 (segment (start 146.5 78.975) (end 155.725 78.975) (width 0.5) (layer "F.Cu") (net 6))
 (segment (start 142.02 77.98) (end 142.5 77.5) (width 0.5) (layer "F.Cu") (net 6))
 (segment (start 155.725 78.975) (end 158.5 81.75) (width 0.5) (layer "F.Cu") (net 6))
 (segment (start 142.02 79) (end 142.02 77.98) (width 0.5) (layer "F.Cu") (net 6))
 (segment (start 140.895 79) (end 142.02 79) (width 0.5) (layer "F.Cu") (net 6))
 (segment (start 136.155 83.74) (end 140.895 79) (width 0.5) (layer "F.Cu") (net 6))
 (segment (start 136.155 85.5) (end 136.155 83.74) (width 0.5) (layer "F.Cu") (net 6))
 (segment (start 125.25 81.39) (end 125.36 81.5) (width 0.4) (layer "F.Cu") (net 3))
 (segment (start 124.5 79.75) (end 124.5 81.39) (width 0.5) (layer "F.Cu") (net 3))
 (segment (start 125.25 79) (end 124.5 79.75) (width 0.5) (layer "F.Cu") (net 3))
 (segment (start 124.5 81.39) (end 125.25 81.39) (width 0.5) (layer "F.Cu") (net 3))
 (segment (start 142 75) (end 142 76) (width 0.5) (layer "F.Cu") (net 10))
 (segment (start 142.5 80.5) (end 142.98 80.02) (width 0.5) (layer "F.Cu") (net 10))
 (segment (start 142.98 80.02) (end 142.98 79) (width 0.5) (layer "F.Cu") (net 10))
 (segment (start 132.5 80.5) (end 131 79) (width 0.5) (layer "F.Cu") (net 10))
 (via (at 142.5 80.5) (size 0.7) (drill 0.3) (layers "F.Cu" "B.Cu") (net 10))
 (via (at 132.5 80.5) (size 0.7) (drill 0.3) (layers "F.Cu" "B.Cu") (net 10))
 (via (at 142 76) (size 0.7) (drill 0.3) (layers "F.Cu" "B.Cu") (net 10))
 (segment (start 142.5 80.5) (end 132.5 80.5) (width 0.5) (layer "B.Cu") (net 10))
 (segment (start 142 80) (end 142.5 80.5) (width 0.5) (layer "B.Cu") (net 10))
 (segment (start 142 76) (end 142 80) (width 0.5) (layer "B.Cu") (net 10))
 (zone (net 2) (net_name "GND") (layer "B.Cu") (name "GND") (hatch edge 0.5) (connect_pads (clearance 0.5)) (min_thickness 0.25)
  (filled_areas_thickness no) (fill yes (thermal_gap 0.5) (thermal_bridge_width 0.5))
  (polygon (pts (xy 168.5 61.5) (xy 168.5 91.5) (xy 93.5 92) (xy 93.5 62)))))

